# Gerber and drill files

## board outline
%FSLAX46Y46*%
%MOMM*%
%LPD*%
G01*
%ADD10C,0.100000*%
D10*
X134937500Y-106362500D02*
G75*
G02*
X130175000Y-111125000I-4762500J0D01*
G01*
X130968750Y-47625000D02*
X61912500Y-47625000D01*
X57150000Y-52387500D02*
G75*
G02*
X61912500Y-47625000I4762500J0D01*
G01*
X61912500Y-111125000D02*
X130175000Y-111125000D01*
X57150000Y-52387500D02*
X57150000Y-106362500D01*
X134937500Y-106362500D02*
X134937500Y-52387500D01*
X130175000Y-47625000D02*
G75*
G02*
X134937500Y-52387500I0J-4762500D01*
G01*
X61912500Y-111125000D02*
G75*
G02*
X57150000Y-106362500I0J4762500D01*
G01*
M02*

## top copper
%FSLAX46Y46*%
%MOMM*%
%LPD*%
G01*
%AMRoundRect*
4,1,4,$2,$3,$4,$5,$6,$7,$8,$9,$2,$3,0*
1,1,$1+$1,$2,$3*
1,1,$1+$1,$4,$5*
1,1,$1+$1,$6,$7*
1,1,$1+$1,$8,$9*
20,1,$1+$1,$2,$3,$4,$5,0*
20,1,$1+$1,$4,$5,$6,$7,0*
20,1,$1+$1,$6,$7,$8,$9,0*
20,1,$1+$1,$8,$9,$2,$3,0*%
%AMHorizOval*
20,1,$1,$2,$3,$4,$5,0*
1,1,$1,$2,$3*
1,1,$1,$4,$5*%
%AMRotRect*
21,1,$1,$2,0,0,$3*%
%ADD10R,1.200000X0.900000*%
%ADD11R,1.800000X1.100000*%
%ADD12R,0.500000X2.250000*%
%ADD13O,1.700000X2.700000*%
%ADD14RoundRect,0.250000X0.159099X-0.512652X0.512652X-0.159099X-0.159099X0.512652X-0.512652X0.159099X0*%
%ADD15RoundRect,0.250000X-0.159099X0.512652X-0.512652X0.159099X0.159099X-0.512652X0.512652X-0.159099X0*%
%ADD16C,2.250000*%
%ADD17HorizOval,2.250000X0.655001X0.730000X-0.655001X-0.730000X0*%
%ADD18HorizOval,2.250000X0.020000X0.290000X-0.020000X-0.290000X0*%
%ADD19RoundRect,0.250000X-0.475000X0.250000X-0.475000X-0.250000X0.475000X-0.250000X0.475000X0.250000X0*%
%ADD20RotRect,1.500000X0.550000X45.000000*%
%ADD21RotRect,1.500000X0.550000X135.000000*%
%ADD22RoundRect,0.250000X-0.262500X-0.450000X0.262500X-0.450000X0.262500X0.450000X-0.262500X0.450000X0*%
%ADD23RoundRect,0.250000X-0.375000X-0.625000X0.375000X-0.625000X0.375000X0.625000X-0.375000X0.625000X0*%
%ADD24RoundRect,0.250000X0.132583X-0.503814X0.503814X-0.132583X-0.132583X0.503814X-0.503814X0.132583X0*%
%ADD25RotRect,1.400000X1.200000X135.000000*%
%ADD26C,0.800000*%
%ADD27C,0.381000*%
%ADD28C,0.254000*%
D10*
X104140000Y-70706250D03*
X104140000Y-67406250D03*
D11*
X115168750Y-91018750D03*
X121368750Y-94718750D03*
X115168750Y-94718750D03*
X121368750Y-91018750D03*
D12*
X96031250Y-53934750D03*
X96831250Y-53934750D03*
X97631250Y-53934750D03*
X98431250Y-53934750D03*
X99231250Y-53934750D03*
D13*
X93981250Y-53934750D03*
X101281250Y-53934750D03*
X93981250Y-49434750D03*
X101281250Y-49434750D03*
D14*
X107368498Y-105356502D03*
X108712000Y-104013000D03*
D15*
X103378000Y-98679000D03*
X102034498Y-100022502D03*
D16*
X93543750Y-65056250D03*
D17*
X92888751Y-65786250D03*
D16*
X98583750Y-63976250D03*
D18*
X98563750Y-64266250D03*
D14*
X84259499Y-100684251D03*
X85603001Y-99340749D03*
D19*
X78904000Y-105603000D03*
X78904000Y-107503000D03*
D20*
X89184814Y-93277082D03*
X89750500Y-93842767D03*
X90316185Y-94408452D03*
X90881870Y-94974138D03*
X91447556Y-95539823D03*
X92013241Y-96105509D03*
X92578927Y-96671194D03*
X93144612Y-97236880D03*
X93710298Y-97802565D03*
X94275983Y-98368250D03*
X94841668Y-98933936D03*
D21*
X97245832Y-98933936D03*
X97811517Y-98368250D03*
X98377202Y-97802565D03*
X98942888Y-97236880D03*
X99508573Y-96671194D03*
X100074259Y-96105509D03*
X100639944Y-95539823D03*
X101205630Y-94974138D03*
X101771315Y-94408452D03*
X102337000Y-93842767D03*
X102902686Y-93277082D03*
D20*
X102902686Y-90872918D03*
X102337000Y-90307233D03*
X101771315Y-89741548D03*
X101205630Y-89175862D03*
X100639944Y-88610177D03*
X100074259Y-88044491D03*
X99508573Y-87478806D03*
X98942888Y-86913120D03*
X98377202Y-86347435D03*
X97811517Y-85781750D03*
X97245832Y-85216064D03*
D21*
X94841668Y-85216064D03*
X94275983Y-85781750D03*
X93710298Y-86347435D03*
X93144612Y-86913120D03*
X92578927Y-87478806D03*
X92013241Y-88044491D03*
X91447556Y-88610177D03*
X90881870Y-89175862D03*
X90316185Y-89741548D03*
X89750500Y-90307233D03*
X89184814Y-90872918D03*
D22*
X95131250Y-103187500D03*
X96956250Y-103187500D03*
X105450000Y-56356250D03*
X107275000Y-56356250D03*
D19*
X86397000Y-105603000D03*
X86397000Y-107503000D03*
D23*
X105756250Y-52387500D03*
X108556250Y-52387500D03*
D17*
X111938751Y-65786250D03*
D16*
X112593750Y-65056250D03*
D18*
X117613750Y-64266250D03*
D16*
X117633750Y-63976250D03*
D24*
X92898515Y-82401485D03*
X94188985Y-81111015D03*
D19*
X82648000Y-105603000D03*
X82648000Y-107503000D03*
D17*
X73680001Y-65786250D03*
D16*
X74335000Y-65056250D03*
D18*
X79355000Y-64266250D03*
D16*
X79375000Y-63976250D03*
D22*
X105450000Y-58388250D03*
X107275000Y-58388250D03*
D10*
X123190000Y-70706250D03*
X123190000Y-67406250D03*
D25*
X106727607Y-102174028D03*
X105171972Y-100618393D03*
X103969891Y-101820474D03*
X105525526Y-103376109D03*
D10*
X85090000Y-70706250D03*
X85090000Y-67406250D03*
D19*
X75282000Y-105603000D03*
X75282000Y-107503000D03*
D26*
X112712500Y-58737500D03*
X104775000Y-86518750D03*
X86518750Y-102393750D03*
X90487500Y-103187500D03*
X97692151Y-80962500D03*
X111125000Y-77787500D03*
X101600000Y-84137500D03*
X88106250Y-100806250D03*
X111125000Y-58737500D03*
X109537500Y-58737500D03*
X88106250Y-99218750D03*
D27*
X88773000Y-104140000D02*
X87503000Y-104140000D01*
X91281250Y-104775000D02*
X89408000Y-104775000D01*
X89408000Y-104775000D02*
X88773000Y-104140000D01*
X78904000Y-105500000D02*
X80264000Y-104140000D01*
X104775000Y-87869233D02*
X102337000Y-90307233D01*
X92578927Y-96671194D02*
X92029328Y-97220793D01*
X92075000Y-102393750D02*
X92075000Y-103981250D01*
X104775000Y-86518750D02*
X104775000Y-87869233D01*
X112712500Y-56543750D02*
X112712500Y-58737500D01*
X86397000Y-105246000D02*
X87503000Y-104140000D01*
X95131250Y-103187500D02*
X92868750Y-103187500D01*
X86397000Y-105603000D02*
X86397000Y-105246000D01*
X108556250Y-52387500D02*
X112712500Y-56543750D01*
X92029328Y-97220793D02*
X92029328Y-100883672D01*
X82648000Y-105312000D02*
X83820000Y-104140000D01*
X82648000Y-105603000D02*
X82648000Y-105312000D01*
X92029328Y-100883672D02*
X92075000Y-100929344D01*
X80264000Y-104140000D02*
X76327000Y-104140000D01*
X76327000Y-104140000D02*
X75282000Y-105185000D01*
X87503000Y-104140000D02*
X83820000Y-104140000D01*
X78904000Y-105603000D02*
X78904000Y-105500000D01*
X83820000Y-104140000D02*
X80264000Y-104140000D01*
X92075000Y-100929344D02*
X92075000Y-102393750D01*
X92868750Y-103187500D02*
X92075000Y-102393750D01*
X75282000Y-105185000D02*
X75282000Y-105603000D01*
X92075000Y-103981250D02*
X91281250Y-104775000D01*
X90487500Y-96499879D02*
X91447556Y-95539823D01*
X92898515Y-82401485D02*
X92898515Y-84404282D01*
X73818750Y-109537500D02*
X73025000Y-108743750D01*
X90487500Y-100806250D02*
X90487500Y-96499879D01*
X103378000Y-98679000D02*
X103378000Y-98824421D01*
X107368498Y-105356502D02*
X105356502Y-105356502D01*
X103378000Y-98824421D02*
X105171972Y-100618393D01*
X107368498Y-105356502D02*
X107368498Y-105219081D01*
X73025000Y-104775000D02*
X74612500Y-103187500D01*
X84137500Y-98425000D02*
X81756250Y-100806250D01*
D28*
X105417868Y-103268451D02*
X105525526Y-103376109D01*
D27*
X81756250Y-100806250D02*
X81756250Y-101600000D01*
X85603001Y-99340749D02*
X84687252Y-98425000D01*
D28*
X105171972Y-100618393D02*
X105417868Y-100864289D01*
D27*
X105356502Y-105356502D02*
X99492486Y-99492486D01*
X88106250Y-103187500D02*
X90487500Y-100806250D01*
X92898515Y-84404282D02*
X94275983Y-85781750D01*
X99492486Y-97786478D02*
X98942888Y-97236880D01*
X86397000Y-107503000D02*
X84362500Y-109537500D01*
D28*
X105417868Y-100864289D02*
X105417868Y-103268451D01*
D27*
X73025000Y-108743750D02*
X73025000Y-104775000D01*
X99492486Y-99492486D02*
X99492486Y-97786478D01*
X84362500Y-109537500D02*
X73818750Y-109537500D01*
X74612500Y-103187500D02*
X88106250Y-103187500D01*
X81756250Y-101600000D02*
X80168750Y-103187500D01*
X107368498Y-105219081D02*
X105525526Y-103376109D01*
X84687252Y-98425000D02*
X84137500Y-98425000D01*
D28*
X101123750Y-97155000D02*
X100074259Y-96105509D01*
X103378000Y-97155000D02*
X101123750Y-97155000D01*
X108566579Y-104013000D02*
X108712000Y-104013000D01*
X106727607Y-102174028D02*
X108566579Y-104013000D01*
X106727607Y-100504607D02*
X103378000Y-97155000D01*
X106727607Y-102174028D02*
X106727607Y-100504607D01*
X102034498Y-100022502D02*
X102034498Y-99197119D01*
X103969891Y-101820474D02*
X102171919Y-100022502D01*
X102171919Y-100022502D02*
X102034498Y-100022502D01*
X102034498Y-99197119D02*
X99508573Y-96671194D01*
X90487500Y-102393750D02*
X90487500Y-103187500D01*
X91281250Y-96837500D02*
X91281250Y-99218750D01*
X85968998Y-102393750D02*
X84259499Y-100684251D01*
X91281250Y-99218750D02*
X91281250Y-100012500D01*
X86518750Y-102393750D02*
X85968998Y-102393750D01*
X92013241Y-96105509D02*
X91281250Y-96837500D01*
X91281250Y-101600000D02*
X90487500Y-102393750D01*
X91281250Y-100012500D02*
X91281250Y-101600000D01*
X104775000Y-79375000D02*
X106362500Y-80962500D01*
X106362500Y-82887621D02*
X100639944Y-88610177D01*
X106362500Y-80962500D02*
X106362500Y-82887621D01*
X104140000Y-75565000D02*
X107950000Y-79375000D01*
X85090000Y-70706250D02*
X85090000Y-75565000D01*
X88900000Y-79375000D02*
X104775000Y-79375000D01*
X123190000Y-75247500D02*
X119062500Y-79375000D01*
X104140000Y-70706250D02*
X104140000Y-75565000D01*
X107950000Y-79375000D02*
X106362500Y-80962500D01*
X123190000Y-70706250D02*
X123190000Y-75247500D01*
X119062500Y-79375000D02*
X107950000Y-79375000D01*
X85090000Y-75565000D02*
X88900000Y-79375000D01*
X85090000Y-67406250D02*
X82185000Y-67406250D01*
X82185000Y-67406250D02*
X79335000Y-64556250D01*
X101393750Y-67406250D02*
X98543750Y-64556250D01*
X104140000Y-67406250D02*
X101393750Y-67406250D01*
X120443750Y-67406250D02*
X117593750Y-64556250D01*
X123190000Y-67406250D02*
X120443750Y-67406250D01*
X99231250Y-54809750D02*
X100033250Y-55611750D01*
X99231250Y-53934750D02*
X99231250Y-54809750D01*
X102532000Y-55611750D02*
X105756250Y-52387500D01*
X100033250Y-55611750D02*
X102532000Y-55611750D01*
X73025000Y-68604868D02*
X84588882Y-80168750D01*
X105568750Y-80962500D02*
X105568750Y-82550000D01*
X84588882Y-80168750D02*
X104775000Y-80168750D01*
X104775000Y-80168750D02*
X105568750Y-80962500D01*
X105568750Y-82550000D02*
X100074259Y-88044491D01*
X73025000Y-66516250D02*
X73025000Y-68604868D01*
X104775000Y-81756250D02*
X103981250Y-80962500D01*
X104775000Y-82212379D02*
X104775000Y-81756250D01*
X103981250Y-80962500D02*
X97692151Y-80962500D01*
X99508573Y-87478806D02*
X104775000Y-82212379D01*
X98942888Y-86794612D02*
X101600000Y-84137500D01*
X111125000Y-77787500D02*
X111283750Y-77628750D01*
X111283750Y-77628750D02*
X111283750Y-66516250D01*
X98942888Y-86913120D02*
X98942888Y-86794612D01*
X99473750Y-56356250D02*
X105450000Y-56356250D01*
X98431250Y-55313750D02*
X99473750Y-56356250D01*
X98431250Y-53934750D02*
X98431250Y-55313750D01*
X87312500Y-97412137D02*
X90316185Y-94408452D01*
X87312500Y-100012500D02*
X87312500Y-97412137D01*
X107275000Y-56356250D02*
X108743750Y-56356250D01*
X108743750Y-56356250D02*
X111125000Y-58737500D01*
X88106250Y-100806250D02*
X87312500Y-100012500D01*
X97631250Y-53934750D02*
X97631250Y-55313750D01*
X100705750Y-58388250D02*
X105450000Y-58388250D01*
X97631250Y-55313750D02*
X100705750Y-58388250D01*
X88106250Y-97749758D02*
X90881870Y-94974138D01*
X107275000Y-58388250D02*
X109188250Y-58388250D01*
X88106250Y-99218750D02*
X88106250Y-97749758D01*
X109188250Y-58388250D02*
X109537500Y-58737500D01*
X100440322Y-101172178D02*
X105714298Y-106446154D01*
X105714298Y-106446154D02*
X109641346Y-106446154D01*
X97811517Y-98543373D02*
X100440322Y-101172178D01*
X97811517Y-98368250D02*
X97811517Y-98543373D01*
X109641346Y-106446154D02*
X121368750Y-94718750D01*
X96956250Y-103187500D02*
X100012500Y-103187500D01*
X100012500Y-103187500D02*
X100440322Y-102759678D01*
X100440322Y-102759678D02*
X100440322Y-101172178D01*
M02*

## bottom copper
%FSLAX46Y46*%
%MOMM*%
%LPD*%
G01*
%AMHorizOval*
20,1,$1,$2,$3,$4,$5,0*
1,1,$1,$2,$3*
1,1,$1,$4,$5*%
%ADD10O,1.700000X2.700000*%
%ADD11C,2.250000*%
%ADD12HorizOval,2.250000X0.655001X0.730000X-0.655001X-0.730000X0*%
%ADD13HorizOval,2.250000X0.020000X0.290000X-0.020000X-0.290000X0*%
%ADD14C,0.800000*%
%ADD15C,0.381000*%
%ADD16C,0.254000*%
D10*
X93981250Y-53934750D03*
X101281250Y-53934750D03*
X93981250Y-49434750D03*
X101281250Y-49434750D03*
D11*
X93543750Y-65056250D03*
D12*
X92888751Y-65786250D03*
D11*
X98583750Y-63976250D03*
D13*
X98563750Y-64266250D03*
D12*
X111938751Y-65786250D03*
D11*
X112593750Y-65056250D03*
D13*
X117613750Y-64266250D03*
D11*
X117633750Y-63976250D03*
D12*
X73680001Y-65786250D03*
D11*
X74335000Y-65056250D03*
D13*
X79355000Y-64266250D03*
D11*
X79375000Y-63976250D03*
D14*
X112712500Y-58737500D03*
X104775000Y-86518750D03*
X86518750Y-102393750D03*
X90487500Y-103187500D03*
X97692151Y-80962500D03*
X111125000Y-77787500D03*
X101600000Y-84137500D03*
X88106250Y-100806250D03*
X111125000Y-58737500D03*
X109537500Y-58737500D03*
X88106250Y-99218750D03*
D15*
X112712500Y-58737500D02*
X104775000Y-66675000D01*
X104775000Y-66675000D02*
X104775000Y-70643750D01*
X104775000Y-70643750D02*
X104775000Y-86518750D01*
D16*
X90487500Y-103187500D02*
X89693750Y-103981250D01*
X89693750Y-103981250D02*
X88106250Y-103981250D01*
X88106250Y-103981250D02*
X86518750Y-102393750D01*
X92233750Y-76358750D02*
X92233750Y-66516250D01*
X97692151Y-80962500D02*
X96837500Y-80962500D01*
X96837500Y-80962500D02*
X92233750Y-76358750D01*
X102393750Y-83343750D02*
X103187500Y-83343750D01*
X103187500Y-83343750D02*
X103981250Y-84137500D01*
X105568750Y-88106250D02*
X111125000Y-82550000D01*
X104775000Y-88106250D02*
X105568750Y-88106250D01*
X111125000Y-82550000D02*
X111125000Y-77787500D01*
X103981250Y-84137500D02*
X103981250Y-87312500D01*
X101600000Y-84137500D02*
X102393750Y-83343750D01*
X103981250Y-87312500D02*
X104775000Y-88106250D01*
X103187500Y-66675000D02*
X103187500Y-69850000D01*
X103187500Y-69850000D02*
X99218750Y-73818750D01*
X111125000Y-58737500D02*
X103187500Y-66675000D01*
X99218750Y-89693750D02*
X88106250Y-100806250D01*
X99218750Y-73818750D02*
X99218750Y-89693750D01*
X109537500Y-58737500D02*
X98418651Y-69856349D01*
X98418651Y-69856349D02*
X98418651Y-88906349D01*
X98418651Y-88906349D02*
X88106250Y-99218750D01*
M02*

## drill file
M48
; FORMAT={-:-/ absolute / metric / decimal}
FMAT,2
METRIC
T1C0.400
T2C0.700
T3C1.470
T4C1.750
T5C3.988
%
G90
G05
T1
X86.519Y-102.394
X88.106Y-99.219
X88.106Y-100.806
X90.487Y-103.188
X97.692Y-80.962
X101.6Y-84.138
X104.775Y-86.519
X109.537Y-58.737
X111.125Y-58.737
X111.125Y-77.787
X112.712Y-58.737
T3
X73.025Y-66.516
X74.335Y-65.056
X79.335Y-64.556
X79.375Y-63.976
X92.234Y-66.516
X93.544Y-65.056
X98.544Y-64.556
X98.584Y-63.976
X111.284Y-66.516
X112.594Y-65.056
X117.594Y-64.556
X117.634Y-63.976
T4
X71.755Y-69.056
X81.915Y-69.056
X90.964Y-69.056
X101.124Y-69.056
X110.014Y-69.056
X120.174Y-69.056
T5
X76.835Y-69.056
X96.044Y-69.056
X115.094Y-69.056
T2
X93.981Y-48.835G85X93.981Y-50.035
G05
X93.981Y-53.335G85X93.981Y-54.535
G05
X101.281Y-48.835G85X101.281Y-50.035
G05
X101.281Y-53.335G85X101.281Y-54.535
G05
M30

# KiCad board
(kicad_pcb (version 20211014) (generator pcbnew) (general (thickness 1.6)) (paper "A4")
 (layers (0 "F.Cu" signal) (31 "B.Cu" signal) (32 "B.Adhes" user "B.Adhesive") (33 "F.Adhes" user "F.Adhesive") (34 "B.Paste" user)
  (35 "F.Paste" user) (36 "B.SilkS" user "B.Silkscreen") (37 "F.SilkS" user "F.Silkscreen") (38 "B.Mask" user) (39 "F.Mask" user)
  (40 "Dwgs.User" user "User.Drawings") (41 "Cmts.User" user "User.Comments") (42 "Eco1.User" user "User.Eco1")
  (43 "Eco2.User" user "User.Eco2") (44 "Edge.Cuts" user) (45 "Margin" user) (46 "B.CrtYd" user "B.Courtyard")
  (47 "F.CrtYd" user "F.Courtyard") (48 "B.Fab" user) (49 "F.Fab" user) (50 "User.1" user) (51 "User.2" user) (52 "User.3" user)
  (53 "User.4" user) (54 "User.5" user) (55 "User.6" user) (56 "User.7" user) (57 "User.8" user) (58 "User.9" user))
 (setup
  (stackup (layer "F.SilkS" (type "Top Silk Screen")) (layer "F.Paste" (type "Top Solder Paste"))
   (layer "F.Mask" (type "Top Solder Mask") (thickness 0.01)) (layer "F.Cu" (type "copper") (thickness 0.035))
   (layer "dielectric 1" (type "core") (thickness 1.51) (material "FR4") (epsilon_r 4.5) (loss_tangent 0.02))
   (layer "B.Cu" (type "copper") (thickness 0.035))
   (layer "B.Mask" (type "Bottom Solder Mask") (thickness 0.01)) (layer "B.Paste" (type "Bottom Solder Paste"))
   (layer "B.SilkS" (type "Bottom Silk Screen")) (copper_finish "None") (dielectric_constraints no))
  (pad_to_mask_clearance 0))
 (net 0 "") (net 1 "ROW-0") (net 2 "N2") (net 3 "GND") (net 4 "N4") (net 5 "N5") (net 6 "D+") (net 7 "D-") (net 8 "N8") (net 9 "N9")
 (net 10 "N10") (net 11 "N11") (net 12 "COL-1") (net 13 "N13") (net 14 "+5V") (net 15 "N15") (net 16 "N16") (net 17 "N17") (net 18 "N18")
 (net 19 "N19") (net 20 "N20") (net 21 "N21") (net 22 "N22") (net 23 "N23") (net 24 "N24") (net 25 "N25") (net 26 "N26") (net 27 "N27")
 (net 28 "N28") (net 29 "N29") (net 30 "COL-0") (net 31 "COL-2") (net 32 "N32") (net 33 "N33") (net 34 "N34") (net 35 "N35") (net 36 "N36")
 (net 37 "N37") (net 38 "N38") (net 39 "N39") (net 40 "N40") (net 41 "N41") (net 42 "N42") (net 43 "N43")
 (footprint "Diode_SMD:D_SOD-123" (layer "F.Cu") (at 104.14 69.05625 90)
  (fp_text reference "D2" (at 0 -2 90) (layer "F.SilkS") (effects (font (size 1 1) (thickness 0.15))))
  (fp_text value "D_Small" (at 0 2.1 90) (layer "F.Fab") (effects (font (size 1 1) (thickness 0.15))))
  (pad "1" smd rect (at -1.65 0 90) (size 0.9 1.2) (layers "F.Cu" "F.Paste" "F.Mask") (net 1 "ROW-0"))
  (pad "2" smd rect (at 1.65 0 90) (size 0.9 1.2) (layers "F.Cu" "F.Paste" "F.Mask") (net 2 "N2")))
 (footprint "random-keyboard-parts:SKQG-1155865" (layer "F.Cu") (at 118.26875 92.86875 180)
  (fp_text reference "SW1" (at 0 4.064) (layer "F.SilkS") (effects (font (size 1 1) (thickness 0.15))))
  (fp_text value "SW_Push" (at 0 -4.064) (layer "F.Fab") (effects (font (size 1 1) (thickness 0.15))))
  (pad "1" smd rect locked (at 3.1 1.85 180) (size 1.8 1.1) (layers "F.Cu" "F.Paste" "F.Mask") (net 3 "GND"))
  (pad "2" smd rect locked (at -3.1 -1.85 180) (size 1.8 1.1) (layers "F.Cu" "F.Paste" "F.Mask") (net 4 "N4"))
  (pad "3" smd rect locked (at 3.1 -1.85 180) (size 1.8 1.1) (layers "F.Cu" "F.Paste" "F.Mask"))
  (pad "4" smd rect locked (at -3.1 1.85 180) (size 1.8 1.1) (layers "F.Cu" "F.Paste" "F.Mask")))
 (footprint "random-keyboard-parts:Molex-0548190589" (layer "F.Cu") (at 97.63125 49.43475 -90)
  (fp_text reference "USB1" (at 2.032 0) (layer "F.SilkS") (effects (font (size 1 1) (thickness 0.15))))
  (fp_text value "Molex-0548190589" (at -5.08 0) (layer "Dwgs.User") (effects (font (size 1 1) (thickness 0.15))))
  (pad "1" smd rect locked (at 4.5 1.6 270) (size 2.25 0.5) (layers "F.Cu" "F.Paste" "F.Mask") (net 3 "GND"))
  (pad "2" smd rect locked (at 4.5 0.8 270) (size 2.25 0.5) (layers "F.Cu" "F.Paste" "F.Mask") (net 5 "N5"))
  (pad "3" smd rect locked (at 4.5 0 270) (size 2.25 0.5) (layers "F.Cu" "F.Paste" "F.Mask") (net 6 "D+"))
  (pad "4" smd rect locked (at 4.5 -0.8 270) (size 2.25 0.5) (layers "F.Cu" "F.Paste" "F.Mask") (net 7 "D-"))
  (pad "5" smd rect locked (at 4.5 -1.6 270) (size 2.25 0.5) (layers "F.Cu" "F.Paste" "F.Mask") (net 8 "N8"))
  (pad "6" thru_hole oval locked (at 4.5 3.65 270) (size 2.7 1.7) (drill oval 1.9 0.7) (layers *.Cu *.Mask) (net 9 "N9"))
  (pad "6" thru_hole oval locked (at 4.5 -3.65 270) (size 2.7 1.7) (drill oval 1.9 0.7) (layers *.Cu *.Mask) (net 9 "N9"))
  (pad "6" thru_hole oval locked (at 0 3.65 270) (size 2.7 1.7) (drill oval 1.9 0.7) (layers *.Cu *.Mask) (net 9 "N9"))
  (pad "6" thru_hole oval locked (at 0 -3.65 270) (size 2.7 1.7) (drill oval 1.9 0.7) (layers *.Cu *.Mask) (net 9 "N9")))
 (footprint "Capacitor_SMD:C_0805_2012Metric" (layer "F.Cu") (at 108.040249 104.684751 45)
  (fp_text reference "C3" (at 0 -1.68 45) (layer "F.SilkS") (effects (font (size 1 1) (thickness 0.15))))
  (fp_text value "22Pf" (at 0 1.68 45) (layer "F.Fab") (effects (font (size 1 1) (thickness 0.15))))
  (pad "1" smd roundrect (at -0.95 0 45) (size 1 1.45) (layers "F.Cu" "F.Paste" "F.Mask") (roundrect_rratio 0.25) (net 3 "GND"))
  (pad "2" smd roundrect (at 0.95 0 45) (size 1 1.45) (layers "F.Cu" "F.Paste" "F.Mask") (roundrect_rratio 0.25) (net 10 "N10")))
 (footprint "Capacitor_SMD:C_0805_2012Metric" (layer "F.Cu") (at 102.706249 99.350751 -135)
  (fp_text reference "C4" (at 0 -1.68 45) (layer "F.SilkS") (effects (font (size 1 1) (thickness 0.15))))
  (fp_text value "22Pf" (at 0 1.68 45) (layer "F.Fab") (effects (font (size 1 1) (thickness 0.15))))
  (pad "1" smd roundrect (at -0.95 0 225) (size 1 1.45) (layers "F.Cu" "F.Paste" "F.Mask") (roundrect_rratio 0.25) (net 3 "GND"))
  (pad "2" smd roundrect (at 0.95 0 225) (size 1 1.45) (layers "F.Cu" "F.Paste" "F.Mask") (roundrect_rratio 0.25) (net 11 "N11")))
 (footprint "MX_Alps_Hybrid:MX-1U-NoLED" (layer "F.Cu") (at 96.04375 69.05625)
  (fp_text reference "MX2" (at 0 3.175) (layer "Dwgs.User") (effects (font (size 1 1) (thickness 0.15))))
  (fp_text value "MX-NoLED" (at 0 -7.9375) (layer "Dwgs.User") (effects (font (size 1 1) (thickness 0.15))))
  (pad "" np_thru_hole circle locked (at -5.08 0 48.0996) (size 1.75 1.75) (drill 1.75) (layers *.Cu *.Mask))
  (pad "" np_thru_hole circle locked (at 0 0) (size 3.9878 3.9878) (drill 3.9878) (layers *.Cu *.Mask))
  (pad "" np_thru_hole circle locked (at 5.08 0 48.0996) (size 1.75 1.75) (drill 1.75) (layers *.Cu *.Mask))
  (pad "1" thru_hole circle locked (at -2.5 -4) (size 2.25 2.25) (drill 1.47) (layers *.Cu "B.Mask") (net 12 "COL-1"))
  (pad "1" thru_hole oval locked (at -3.81 -2.54 48.0996) (size 4.211556 2.25) (drill 1.47 (offset 0.980778 0)) (layers *.Cu "B.Mask")
   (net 12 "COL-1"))
  (pad "2" thru_hole circle locked (at 2.54 -5.08) (size 2.25 2.25) (drill 1.47) (layers *.Cu "B.Mask") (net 2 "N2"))
  (pad "2" thru_hole oval locked (at 2.5 -4.5 86.0548) (size 2.831378 2.25) (drill 1.47 (offset 0.290689 0)) (layers *.Cu "B.Mask")
   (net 2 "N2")))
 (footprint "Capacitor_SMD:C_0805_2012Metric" (layer "F.Cu") (at 84.93125 100.0125 45)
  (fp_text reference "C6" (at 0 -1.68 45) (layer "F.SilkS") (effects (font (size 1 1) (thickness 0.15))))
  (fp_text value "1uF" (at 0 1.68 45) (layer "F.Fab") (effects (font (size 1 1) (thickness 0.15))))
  (pad "1" smd roundrect (at -0.95 0 45) (size 1 1.45) (layers "F.Cu" "F.Paste" "F.Mask") (roundrect_rratio 0.25) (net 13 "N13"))
  (pad "2" smd roundrect (at 0.95 0 45) (size 1 1.45) (layers "F.Cu" "F.Paste" "F.Mask") (roundrect_rratio 0.25) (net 3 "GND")))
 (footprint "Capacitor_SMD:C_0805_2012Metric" (layer "F.Cu") (at 78.904 106.553 -90)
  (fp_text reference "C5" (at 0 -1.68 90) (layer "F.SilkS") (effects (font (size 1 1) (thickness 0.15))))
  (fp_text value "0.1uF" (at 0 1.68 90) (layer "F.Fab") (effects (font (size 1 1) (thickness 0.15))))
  (pad "1" smd roundrect (at -0.95 0 270) (size 1 1.45) (layers "F.Cu" "F.Paste" "F.Mask") (roundrect_rratio 0.25) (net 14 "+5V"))
  (pad "2" smd roundrect (at 0.95 0 270) (size 1 1.45) (layers "F.Cu" "F.Paste" "F.Mask") (roundrect_rratio 0.25) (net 3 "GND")))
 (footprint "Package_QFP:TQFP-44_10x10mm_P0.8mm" (layer "F.Cu") (at 96.04375 92.075 45)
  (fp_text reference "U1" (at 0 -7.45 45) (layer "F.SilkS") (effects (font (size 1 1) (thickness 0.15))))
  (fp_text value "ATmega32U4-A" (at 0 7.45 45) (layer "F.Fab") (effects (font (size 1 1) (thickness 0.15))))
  (pad "1" smd rect (at -5.7 -4 45) (size 1.5 0.55) (layers "F.Cu" "F.Paste" "F.Mask") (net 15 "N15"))
  (pad "2" smd rect (at -5.7 -3.2 45) (size 1.5 0.55) (layers "F.Cu" "F.Paste" "F.Mask") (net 14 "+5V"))
  (pad "3" smd rect (at -5.7 -2.4 45) (size 1.5 0.55) (layers "F.Cu" "F.Paste" "F.Mask") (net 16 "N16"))
  (pad "4" smd rect (at -5.7 -1.6 45) (size 1.5 0.55) (layers "F.Cu" "F.Paste" "F.Mask") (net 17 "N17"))
  (pad "5" smd rect (at -5.7 -0.8 45) (size 1.5 0.55) (layers "F.Cu" "F.Paste" "F.Mask") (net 3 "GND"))
  (pad "6" smd rect (at -5.7 0 45) (size 1.5 0.55) (layers "F.Cu" "F.Paste" "F.Mask") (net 13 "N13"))
  (pad "7" smd rect (at -5.7 0.8 45) (size 1.5 0.55) (layers "F.Cu" "F.Paste" "F.Mask") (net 14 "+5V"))
  (pad "8" smd rect (at -5.7 1.6 45) (size 1.5 0.55) (layers "F.Cu" "F.Paste" "F.Mask") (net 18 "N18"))
  (pad "9" smd rect (at -5.7 2.4 45) (size 1.5 0.55) (layers "F.Cu" "F.Paste" "F.Mask") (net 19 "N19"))
  (pad "10" smd rect (at -5.7 3.2 45) (size 1.5 0.55) (layers "F.Cu" "F.Paste" "F.Mask") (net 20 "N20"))
  (pad "11" smd rect (at -5.7 4 45) (size 1.5 0.55) (layers "F.Cu" "F.Paste" "F.Mask") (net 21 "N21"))
  (pad "12" smd rect (at -4 5.7 135) (size 1.5 0.55) (layers "F.Cu" "F.Paste" "F.Mask") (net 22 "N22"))
  (pad "13" smd rect (at -3.2 5.7 135) (size 1.5 0.55) (layers "F.Cu" "F.Paste" "F.Mask") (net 4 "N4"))
  (pad "14" smd rect (at -2.4 5.7 135) (size 1.5 0.55) (layers "F.Cu" "F.Paste" "F.Mask") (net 14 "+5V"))
  (pad "15" smd rect (at -1.6 5.7 135) (size 1.5 0.55) (layers "F.Cu" "F.Paste" "F.Mask") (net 3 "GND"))
  (pad "16" smd rect (at -0.8 5.7 135) (size 1.5 0.55) (layers "F.Cu" "F.Paste" "F.Mask") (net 11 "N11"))
  (pad "17" smd rect (at 0 5.7 135) (size 1.5 0.55) (layers "F.Cu" "F.Paste" "F.Mask") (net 10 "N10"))
  (pad "18" smd rect (at 0.8 5.7 135) (size 1.5 0.55) (layers "F.Cu" "F.Paste" "F.Mask") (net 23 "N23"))
  (pad "19" smd rect (at 1.6 5.7 135) (size 1.5 0.55) (layers "F.Cu" "F.Paste" "F.Mask") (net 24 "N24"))
  (pad "20" smd rect (at 2.4 5.7 135) (size 1.5 0.55) (layers "F.Cu" "F.Paste" "F.Mask") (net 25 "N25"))
  (pad "21" smd rect (at 3.2 5.7 135) (size 1.5 0.55) (layers "F.Cu" "F.Paste" "F.Mask") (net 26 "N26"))
  (pad "22" smd rect (at 4 5.7 135) (size 1.5 0.55) (layers "F.Cu" "F.Paste" "F.Mask") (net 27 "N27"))
  (pad "23" smd rect (at 5.7 4 45) (size 1.5 0.55) (layers "F.Cu" "F.Paste" "F.Mask") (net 3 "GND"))
  (pad "24" smd rect (at 5.7 3.2 45) (size 1.5 0.55) (layers "F.Cu" "F.Paste" "F.Mask") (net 14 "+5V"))
  (pad "25" smd rect (at 5.7 2.4 45) (size 1.5 0.55) (layers "F.Cu" "F.Paste" "F.Mask") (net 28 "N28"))
  (pad "26" smd rect (at 5.7 1.6 45) (size 1.5 0.55) (layers "F.Cu" "F.Paste" "F.Mask") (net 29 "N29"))
  (pad "27" smd rect (at 5.7 0.8 45) (size 1.5 0.55) (layers "F.Cu" "F.Paste" "F.Mask") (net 1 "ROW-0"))
  (pad "28" smd rect (at 5.7 0 45) (size 1.5 0.55) (layers "F.Cu" "F.Paste" "F.Mask") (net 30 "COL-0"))
  (pad "29" smd rect (at 5.7 -0.8 45) (size 1.5 0.55) (layers "F.Cu" "F.Paste" "F.Mask") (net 12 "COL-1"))
  (pad "30" smd rect (at 5.7 -1.6 45) (size 1.5 0.55) (layers "F.Cu" "F.Paste" "F.Mask") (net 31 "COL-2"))
  (pad "31" smd rect (at 5.7 -2.4 45) (size 1.5 0.55) (layers "F.Cu" "F.Paste" "F.Mask") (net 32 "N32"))
  (pad "32" smd rect (at 5.7 -3.2 45) (size 1.5 0.55) (layers "F.Cu" "F.Paste" "F.Mask") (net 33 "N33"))
  (pad "33" smd rect (at 5.7 -4 45) (size 1.5 0.55) (layers "F.Cu" "F.Paste" "F.Mask") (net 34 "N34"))
  (pad "34" smd rect (at 4 -5.7 135) (size 1.5 0.55) (layers "F.Cu" "F.Paste" "F.Mask") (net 14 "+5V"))
  (pad "35" smd rect (at 3.2 -5.7 135) (size 1.5 0.55) (layers "F.Cu" "F.Paste" "F.Mask") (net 3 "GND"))
  (pad "36" smd rect (at 2.4 -5.7 135) (size 1.5 0.55) (layers "F.Cu" "F.Paste" "F.Mask") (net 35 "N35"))
  (pad "37" smd rect (at 1.6 -5.7 135) (size 1.5 0.55) (layers "F.Cu" "F.Paste" "F.Mask") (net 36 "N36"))
  (pad "38" smd rect (at 0.8 -5.7 135) (size 1.5 0.55) (layers "F.Cu" "F.Paste" "F.Mask") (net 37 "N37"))
  (pad "39" smd rect (at 0 -5.7 135) (size 1.5 0.55) (layers "F.Cu" "F.Paste" "F.Mask") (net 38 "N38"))
  (pad "40" smd rect (at -0.8 -5.7 135) (size 1.5 0.55) (layers "F.Cu" "F.Paste" "F.Mask") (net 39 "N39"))
  (pad "41" smd rect (at -1.6 -5.7 135) (size 1.5 0.55) (layers "F.Cu" "F.Paste" "F.Mask") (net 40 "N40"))
  (pad "42" smd rect (at -2.4 -5.7 135) (size 1.5 0.55) (layers "F.Cu" "F.Paste" "F.Mask") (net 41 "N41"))
  (pad "43" smd rect (at -3.2 -5.7 135) (size 1.5 0.55) (layers "F.Cu" "F.Paste" "F.Mask") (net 3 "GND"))
  (pad "44" smd rect (at -4 -5.7 135) (size 1.5 0.55) (layers "F.Cu" "F.Paste" "F.Mask") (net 14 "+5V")))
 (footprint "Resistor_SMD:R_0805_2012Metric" (layer "F.Cu") (at 96.04375 103.1875)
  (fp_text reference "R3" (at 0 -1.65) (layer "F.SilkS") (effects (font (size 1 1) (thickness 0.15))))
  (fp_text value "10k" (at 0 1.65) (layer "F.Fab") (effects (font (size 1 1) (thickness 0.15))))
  (pad "1" smd roundrect (at -0.9125 0) (size 1.025 1.4) (layers "F.Cu" "F.Paste" "F.Mask") (roundrect_rratio 0.243902) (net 14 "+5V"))
  (pad "2" smd roundrect (at 0.9125 0) (size 1.025 1.4) (layers "F.Cu" "F.Paste" "F.Mask") (roundrect_rratio 0.243902) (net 4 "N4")))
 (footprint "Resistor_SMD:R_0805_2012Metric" (layer "F.Cu") (at 106.3625 56.35625)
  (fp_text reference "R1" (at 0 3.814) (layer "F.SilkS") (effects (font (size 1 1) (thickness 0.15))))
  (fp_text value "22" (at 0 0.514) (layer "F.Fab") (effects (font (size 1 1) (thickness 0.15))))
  (pad "1" smd roundrect (at -0.9125 0) (size 1.025 1.4) (layers "F.Cu" "F.Paste" "F.Mask") (roundrect_rratio 0.243902) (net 7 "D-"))
  (pad "2" smd roundrect (at 0.9125 0) (size 1.025 1.4) (layers "F.Cu" "F.Paste" "F.Mask") (roundrect_rratio 0.243902) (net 16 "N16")))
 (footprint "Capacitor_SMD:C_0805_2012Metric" (layer "F.Cu") (at 86.397 106.553 -90)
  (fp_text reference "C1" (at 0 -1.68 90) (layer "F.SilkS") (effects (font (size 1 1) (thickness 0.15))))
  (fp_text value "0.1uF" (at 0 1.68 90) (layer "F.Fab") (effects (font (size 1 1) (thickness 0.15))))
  (pad "1" smd roundrect (at -0.95 0 270) (size 1 1.45) (layers "F.Cu" "F.Paste" "F.Mask") (roundrect_rratio 0.25) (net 14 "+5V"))
  (pad "2" smd roundrect (at 0.95 0 270) (size 1 1.45) (layers "F.Cu" "F.Paste" "F.Mask") (roundrect_rratio 0.25) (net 3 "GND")))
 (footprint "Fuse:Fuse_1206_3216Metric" (layer "F.Cu") (at 107.15625 52.3875)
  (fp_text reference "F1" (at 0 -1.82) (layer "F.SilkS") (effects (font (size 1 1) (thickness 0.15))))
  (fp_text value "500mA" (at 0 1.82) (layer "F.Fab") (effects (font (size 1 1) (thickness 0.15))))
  (pad "1" smd roundrect (at -1.4 0) (size 1.25 1.75) (layers "F.Cu" "F.Paste" "F.Mask") (roundrect_rratio 0.2) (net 8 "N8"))
  (pad "2" smd roundrect (at 1.4 0) (size 1.25 1.75) (layers "F.Cu" "F.Paste" "F.Mask") (roundrect_rratio 0.2) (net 14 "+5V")))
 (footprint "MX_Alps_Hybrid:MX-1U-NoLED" (layer "F.Cu") (at 115.09375 69.05625)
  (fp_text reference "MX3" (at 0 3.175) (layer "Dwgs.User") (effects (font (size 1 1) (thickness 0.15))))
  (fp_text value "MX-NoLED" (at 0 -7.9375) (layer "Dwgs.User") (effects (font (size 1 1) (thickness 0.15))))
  (pad "" np_thru_hole circle locked (at -5.08 0 48.0996) (size 1.75 1.75) (drill 1.75) (layers *.Cu *.Mask))
  (pad "" np_thru_hole circle locked (at 5.08 0 48.0996) (size 1.75 1.75) (drill 1.75) (layers *.Cu *.Mask))
  (pad "" np_thru_hole circle locked (at 0 0) (size 3.9878 3.9878) (drill 3.9878) (layers *.Cu *.Mask))
  (pad "1" thru_hole oval locked (at -3.81 -2.54 48.0996) (size 4.211556 2.25) (drill 1.47 (offset 0.980778 0)) (layers *.Cu "B.Mask")
   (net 31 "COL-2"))
  (pad "1" thru_hole circle locked (at -2.5 -4) (size 2.25 2.25) (drill 1.47) (layers *.Cu "B.Mask") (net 31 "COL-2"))
  (pad "2" thru_hole oval locked (at 2.5 -4.5 86.0548) (size 2.831378 2.25) (drill 1.47 (offset 0.290689 0)) (layers *.Cu "B.Mask")
   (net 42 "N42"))
  (pad "2" thru_hole circle locked (at 2.54 -5.08) (size 2.25 2.25) (drill 1.47) (layers *.Cu "B.Mask") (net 42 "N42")))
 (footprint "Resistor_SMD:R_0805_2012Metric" (layer "F.Cu") (at 93.54375 81.75625 45)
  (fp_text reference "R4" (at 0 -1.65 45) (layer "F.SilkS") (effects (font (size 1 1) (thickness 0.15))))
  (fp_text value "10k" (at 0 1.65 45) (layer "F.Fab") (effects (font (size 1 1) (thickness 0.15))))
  (pad "1" smd roundrect (at -0.9125 0 45) (size 1.025 1.4) (layers "F.Cu" "F.Paste" "F.Mask") (roundrect_rratio 0.243902) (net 3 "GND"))
  (pad "2" smd roundrect (at 0.9125 0 45) (size 1.025 1.4) (layers "F.Cu" "F.Paste" "F.Mask") (roundrect_rratio 0.243902) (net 34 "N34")))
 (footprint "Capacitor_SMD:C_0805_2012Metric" (layer "F.Cu") (at 82.648 106.553 -90)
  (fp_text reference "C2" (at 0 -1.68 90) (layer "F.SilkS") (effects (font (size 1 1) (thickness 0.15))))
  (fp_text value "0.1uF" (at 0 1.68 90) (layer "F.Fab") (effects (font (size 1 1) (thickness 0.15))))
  (pad "1" smd roundrect (at -0.95 0 270) (size 1 1.45) (layers "F.Cu" "F.Paste" "F.Mask") (roundrect_rratio 0.25) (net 14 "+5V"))
  (pad "2" smd roundrect (at 0.95 0 270) (size 1 1.45) (layers "F.Cu" "F.Paste" "F.Mask") (roundrect_rratio 0.25) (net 3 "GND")))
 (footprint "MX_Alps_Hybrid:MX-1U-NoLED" (layer "F.Cu") (at 76.835 69.05625)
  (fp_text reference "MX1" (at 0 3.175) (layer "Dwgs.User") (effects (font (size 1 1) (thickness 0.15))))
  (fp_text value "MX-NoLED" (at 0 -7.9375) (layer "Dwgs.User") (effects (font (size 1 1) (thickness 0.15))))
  (pad "" np_thru_hole circle locked (at -5.08 0 48.0996) (size 1.75 1.75) (drill 1.75) (layers *.Cu *.Mask))
  (pad "" np_thru_hole circle locked (at 5.08 0 48.0996) (size 1.75 1.75) (drill 1.75) (layers *.Cu *.Mask))
  (pad "" np_thru_hole circle locked (at 0 0) (size 3.9878 3.9878) (drill 3.9878) (layers *.Cu *.Mask))
  (pad "1" thru_hole oval locked (at -3.81 -2.54 48.0996) (size 4.211556 2.25) (drill 1.47 (offset 0.980778 0)) (layers *.Cu "B.Mask")
   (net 30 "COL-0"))
  (pad "1" thru_hole circle locked (at -2.5 -4) (size 2.25 2.25) (drill 1.47) (layers *.Cu "B.Mask") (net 30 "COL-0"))
  (pad "2" thru_hole oval locked (at 2.5 -4.5 86.0548) (size 2.831378 2.25) (drill 1.47 (offset 0.290689 0)) (layers *.Cu "B.Mask")
   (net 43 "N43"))
  (pad "2" thru_hole circle locked (at 2.54 -5.08) (size 2.25 2.25) (drill 1.47) (layers *.Cu "B.Mask") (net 43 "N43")))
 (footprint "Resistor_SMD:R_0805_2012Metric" (layer "F.Cu") (at 106.3625 58.38825)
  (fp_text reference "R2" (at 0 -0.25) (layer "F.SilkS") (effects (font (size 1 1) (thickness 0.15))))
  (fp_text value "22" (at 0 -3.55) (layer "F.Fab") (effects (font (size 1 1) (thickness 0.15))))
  (pad "1" smd roundrect (at -0.9125 0) (size 1.025 1.4) (layers "F.Cu" "F.Paste" "F.Mask") (roundrect_rratio 0.243902) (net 6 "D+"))
  (pad "2" smd roundrect (at 0.9125 0) (size 1.025 1.4) (layers "F.Cu" "F.Paste" "F.Mask") (roundrect_rratio 0.243902) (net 17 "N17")))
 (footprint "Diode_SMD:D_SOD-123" (layer "F.Cu") (at 123.19 69.05625 90)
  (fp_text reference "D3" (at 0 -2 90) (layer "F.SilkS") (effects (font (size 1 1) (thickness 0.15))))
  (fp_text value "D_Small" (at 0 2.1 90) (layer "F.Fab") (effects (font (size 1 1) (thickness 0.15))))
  (pad "1" smd rect (at -1.65 0 90) (size 0.9 1.2) (layers "F.Cu" "F.Paste" "F.Mask") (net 1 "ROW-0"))
  (pad "2" smd rect (at 1.65 0 90) (size 0.9 1.2) (layers "F.Cu" "F.Paste" "F.Mask") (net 42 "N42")))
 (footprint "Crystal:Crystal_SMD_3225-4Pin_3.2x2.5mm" (layer "F.Cu") (at 105.348749 101.997251 135)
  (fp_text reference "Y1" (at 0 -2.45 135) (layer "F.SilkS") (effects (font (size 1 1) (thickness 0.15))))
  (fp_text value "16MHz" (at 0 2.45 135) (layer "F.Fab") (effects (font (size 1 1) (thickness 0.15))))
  (pad "1" smd rect (at -1.1 0.85 135) (size 1.4 1.2) (layers "F.Cu" "F.Paste" "F.Mask") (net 10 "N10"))
  (pad "2" smd rect (at 1.1 0.85 135) (size 1.4 1.2) (layers "F.Cu" "F.Paste" "F.Mask") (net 3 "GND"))
  (pad "3" smd rect (at 1.1 -0.85 135) (size 1.4 1.2) (layers "F.Cu" "F.Paste" "F.Mask") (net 11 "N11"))
  (pad "4" smd rect (at -1.1 -0.85 135) (size 1.4 1.2) (layers "F.Cu" "F.Paste" "F.Mask") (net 3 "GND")))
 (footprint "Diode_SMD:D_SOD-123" (layer "F.Cu") (at 85.09 69.05625 90)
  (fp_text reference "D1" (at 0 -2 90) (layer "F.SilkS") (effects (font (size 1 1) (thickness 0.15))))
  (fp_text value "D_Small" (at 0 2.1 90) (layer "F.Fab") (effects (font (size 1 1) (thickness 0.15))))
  (pad "1" smd rect (at -1.65 0 90) (size 0.9 1.2) (layers "F.Cu" "F.Paste" "F.Mask") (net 1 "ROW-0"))
  (pad "2" smd rect (at 1.65 0 90) (size 0.9 1.2) (layers "F.Cu" "F.Paste" "F.Mask") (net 43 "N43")))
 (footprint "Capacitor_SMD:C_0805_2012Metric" (layer "F.Cu") (at 75.282 106.553 -90)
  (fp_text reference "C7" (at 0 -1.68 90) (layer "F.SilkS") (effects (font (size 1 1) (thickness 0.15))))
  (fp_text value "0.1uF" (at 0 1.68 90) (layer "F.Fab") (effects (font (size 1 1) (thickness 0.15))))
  (pad "1" smd roundrect (at -0.95 0 270) (size 1 1.45) (layers "F.Cu" "F.Paste" "F.Mask") (roundrect_rratio 0.25) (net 14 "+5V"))
  (pad "2" smd roundrect (at 0.95 0 270) (size 1 1.45) (layers "F.Cu" "F.Paste" "F.Mask") (roundrect_rratio 0.25) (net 3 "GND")))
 (gr_arc (start 134.9375 106.3625) (mid 133.542596 109.730096) (end 130.175 111.125) (layer "Edge.Cuts") (width 0.1))
 (gr_line (start 130.96875 47.625) (end 61.9125 47.625) (layer "Edge.Cuts") (width 0.1))
 (gr_arc (start 57.15 52.3875) (mid 58.544904 49.019904) (end 61.9125 47.625) (layer "Edge.Cuts") (width 0.1))
 (gr_line (start 61.9125 111.125) (end 130.175 111.125) (layer "Edge.Cuts") (width 0.1))
 (gr_line (start 57.15 52.3875) (end 57.15 106.3625) (layer "Edge.Cuts") (width 0.1))
 (gr_line (start 134.9375 106.3625) (end 134.9375 52.3875) (layer "Edge.Cuts") (width 0.1))
 (gr_arc (start 130.175 47.625) (mid 133.542596 49.019904) (end 134.9375 52.3875) (layer "Edge.Cuts") (width 0.1))
 (gr_arc (start 61.9125 111.125) (mid 58.544904 109.730096) (end 57.15 106.3625) (layer "Edge.Cuts") (width 0.1))
 (segment (start 88.773 104.14) (end 87.503 104.14) (width 0.381) (layer "F.Cu") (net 14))
 (segment (start 91.28125 104.775) (end 89.408 104.775) (width 0.381) (layer "F.Cu") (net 14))
 (segment (start 89.408 104.775) (end 88.773 104.14) (width 0.381) (layer "F.Cu") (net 14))
 (segment (start 78.904 105.5) (end 80.264 104.14) (width 0.381) (layer "F.Cu") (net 14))
 (segment (start 104.775 87.869233) (end 102.337 90.307233) (width 0.381) (layer "F.Cu") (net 14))
 (segment (start 92.578927 96.671194) (end 92.029328 97.220793) (width 0.381) (layer "F.Cu") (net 14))
 (segment (start 92.075 102.39375) (end 92.075 103.98125) (width 0.381) (layer "F.Cu") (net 14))
 (segment (start 104.775 86.51875) (end 104.775 87.869233) (width 0.381) (layer "F.Cu") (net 14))
 (segment (start 112.7125 56.54375) (end 112.7125 58.7375) (width 0.381) (layer "F.Cu") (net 14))
 (segment (start 86.397 105.246) (end 87.503 104.14) (width 0.381) (layer "F.Cu") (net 14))
 (segment (start 95.13125 103.1875) (end 92.86875 103.1875) (width 0.381) (layer "F.Cu") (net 14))
 (segment (start 86.397 105.603) (end 86.397 105.246) (width 0.381) (layer "F.Cu") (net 14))
 (segment (start 108.55625 52.3875) (end 112.7125 56.54375) (width 0.381) (layer "F.Cu") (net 14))
 (segment (start 92.029328 97.220793) (end 92.029328 100.883672) (width 0.381) (layer "F.Cu") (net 14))
 (segment (start 82.648 105.312) (end 83.82 104.14) (width 0.381) (layer "F.Cu") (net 14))
 (segment (start 82.648 105.603) (end 82.648 105.312) (width 0.381) (layer "F.Cu") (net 14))
 (segment (start 92.029328 100.883672) (end 92.075 100.929344) (width 0.381) (layer "F.Cu") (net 14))
 (segment (start 80.264 104.14) (end 76.327 104.14) (width 0.381) (layer "F.Cu") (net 14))
 (segment (start 76.327 104.14) (end 75.282 105.185) (width 0.381) (layer "F.Cu") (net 14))
 (segment (start 87.503 104.14) (end 83.82 104.14) (width 0.381) (layer "F.Cu") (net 14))
 (segment (start 78.904 105.603) (end 78.904 105.5) (width 0.381) (layer "F.Cu") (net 14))
 (segment (start 83.82 104.14) (end 80.264 104.14) (width 0.381) (layer "F.Cu") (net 14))
 (segment (start 92.075 100.929344) (end 92.075 102.39375) (width 0.381) (layer "F.Cu") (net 14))
 (segment (start 92.86875 103.1875) (end 92.075 102.39375) (width 0.381) (layer "F.Cu") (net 14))
 (segment (start 75.282 105.185) (end 75.282 105.603) (width 0.381) (layer "F.Cu") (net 14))
 (segment (start 92.075 103.98125) (end 91.28125 104.775) (width 0.381) (layer "F.Cu") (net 14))
 (via (at 112.7125 58.7375) (size 0.8) (drill 0.4) (layers "F.Cu" "B.Cu") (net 14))
 (via (at 104.775 86.51875) (size 0.8) (drill 0.4) (layers "F.Cu" "B.Cu") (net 14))
 (segment (start 112.7125 58.7375) (end 104.775 66.675) (width 0.381) (layer "B.Cu") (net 14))
 (segment (start 104.775 66.675) (end 104.775 70.64375) (width 0.381) (layer "B.Cu") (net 14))
 (segment (start 104.775 70.64375) (end 104.775 86.51875) (width 0.381) (layer "B.Cu") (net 14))
 (segment (start 90.4875 96.499879) (end 91.447556 95.539823) (width 0.381) (layer "F.Cu") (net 3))
 (segment (start 92.898515 82.401485) (end 92.898515 84.404282) (width 0.381) (layer "F.Cu") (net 3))
 (segment (start 73.81875 109.5375) (end 73.025 108.74375) (width 0.381) (layer "F.Cu") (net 3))
 (segment (start 90.4875 100.80625) (end 90.4875 96.499879) (width 0.381) (layer "F.Cu") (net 3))
 (segment (start 103.378 98.679) (end 103.378 98.824421) (width 0.381) (layer "F.Cu") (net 3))
 (segment (start 107.368498 105.356502) (end 105.356502 105.356502) (width 0.381) (layer "F.Cu") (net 3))
 (segment (start 103.378 98.824421) (end 105.171972 100.618393) (width 0.381) (layer "F.Cu") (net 3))
 (segment (start 107.368498 105.356502) (end 107.368498 105.219081) (width 0.381) (layer "F.Cu") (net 3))
 (segment (start 73.025 104.775) (end 74.6125 103.1875) (width 0.381) (layer "F.Cu") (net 3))
 (segment (start 84.1375 98.425) (end 81.75625 100.80625) (width 0.381) (layer "F.Cu") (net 3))
 (segment (start 105.417868 103.268451) (end 105.525526 103.376109) (width 0.254) (layer "F.Cu") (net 3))
 (segment (start 81.75625 100.80625) (end 81.75625 101.6) (width 0.381) (layer "F.Cu") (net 3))
 (segment (start 85.603001 99.340749) (end 84.687252 98.425) (width 0.381) (layer "F.Cu") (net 3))
 (segment (start 105.171972 100.618393) (end 105.417868 100.864289) (width 0.254) (layer "F.Cu") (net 3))
 (segment (start 105.356502 105.356502) (end 99.492486 99.492486) (width 0.381) (layer "F.Cu") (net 3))
 (segment (start 88.10625 103.1875) (end 90.4875 100.80625) (width 0.381) (layer "F.Cu") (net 3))
 (segment (start 92.898515 84.404282) (end 94.275983 85.78175) (width 0.381) (layer "F.Cu") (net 3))
 (segment (start 99.492486 97.786478) (end 98.942888 97.23688) (width 0.381) (layer "F.Cu") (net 3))
 (segment (start 86.397 107.503) (end 84.3625 109.5375) (width 0.381) (layer "F.Cu") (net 3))
 (segment (start 105.417868 100.864289) (end 105.417868 103.268451) (width 0.254) (layer "F.Cu") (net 3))
 (segment (start 73.025 108.74375) (end 73.025 104.775) (width 0.381) (layer "F.Cu") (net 3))
 (segment (start 99.492486 99.492486) (end 99.492486 97.786478) (width 0.381) (layer "F.Cu") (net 3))
 (segment (start 84.3625 109.5375) (end 73.81875 109.5375) (width 0.381) (layer "F.Cu") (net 3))
 (segment (start 74.6125 103.1875) (end 88.10625 103.1875) (width 0.381) (layer "F.Cu") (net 3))
 (segment (start 81.75625 101.6) (end 80.16875 103.1875) (width 0.381) (layer "F.Cu") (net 3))
 (segment (start 107.368498 105.219081) (end 105.525526 103.376109) (width 0.381) (layer "F.Cu") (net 3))
 (segment (start 84.687252 98.425) (end 84.1375 98.425) (width 0.381) (layer "F.Cu") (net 3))
 (segment (start 101.12375 97.155) (end 100.074259 96.105509) (width 0.254) (layer "F.Cu") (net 10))
 (segment (start 103.378 97.155) (end 101.12375 97.155) (width 0.254) (layer "F.Cu") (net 10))
 (segment (start 108.566579 104.013) (end 108.712 104.013) (width 0.254) (layer "F.Cu") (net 10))
 (segment (start 106.727607 102.174028) (end 108.566579 104.013) (width 0.254) (layer "F.Cu") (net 10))
 (segment (start 106.727607 100.504607) (end 103.378 97.155) (width 0.254) (layer "F.Cu") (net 10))
 (segment (start 106.727607 102.174028) (end 106.727607 100.504607) (width 0.254) (layer "F.Cu") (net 10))
 (segment (start 102.034498 100.022502) (end 102.034498 99.197119) (width 0.254) (layer "F.Cu") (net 11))
 (segment (start 103.969891 101.820474) (end 102.171919 100.022502) (width 0.254) (layer "F.Cu") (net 11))
 (segment (start 102.171919 100.022502) (end 102.034498 100.022502) (width 0.254) (layer "F.Cu") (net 11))
 (segment (start 102.034498 99.197119) (end 99.508573 96.671194) (width 0.254) (layer "F.Cu") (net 11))
 (segment (start 90.4875 102.39375) (end 90.4875 103.1875) (width 0.254) (layer "F.Cu") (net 13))
 (segment (start 91.28125 96.8375) (end 91.28125 99.21875) (width 0.254) (layer "F.Cu") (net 13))
 (segment (start 85.968998 102.39375) (end 84.259499 100.684251) (width 0.254) (layer "F.Cu") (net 13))
 (segment (start 91.28125 99.21875) (end 91.28125 100.0125) (width 0.254) (layer "F.Cu") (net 13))
 (segment (start 86.51875 102.39375) (end 85.968998 102.39375) (width 0.254) (layer "F.Cu") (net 13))
 (segment (start 92.013241 96.105509) (end 91.28125 96.8375) (width 0.254) (layer "F.Cu") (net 13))
 (segment (start 91.28125 101.6) (end 90.4875 102.39375) (width 0.254) (layer "F.Cu") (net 13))
 (segment (start 91.28125 100.0125) (end 91.28125 101.6) (width 0.254) (layer "F.Cu") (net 13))
 (via (at 86.51875 102.39375) (size 0.8) (drill 0.4) (layers "F.Cu" "B.Cu") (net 13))
 (via (at 90.4875 103.1875) (size 0.8) (drill 0.4) (layers "F.Cu" "B.Cu") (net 13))
 (segment (start 90.4875 103.1875) (end 89.69375 103.98125) (width 0.254) (layer "B.Cu") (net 13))
 (segment (start 89.69375 103.98125) (end 88.10625 103.98125) (width 0.254) (layer "B.Cu") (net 13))
 (segment (start 88.10625 103.98125) (end 86.51875 102.39375) (width 0.254) (layer "B.Cu") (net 13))
 (segment (start 104.775 79.375) (end 106.3625 80.9625) (width 0.254) (layer "F.Cu") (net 1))
 (segment (start 106.3625 82.887621) (end 100.639944 88.610177) (width 0.254) (layer "F.Cu") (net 1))
 (segment (start 106.3625 80.9625) (end 106.3625 82.887621) (width 0.254) (layer "F.Cu") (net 1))
 (segment (start 104.14 75.565) (end 107.95 79.375) (width 0.254) (layer "F.Cu") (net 1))
 (segment (start 85.09 70.70625) (end 85.09 75.565) (width 0.254) (layer "F.Cu") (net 1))
 (segment (start 88.9 79.375) (end 104.775 79.375) (width 0.254) (layer "F.Cu") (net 1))
 (segment (start 123.19 75.2475) (end 119.0625 79.375) (width 0.254) (layer "F.Cu") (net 1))
 (segment (start 104.14 70.70625) (end 104.14 75.565) (width 0.254) (layer "F.Cu") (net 1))
 (segment (start 107.95 79.375) (end 106.3625 80.9625) (width 0.254) (layer "F.Cu") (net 1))
 (segment (start 123.19 70.70625) (end 123.19 75.2475) (width 0.254) (layer "F.Cu") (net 1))
 (segment (start 119.0625 79.375) (end 107.95 79.375) (width 0.254) (layer "F.Cu") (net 1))
 (segment (start 85.09 75.565) (end 88.9 79.375) (width 0.254) (layer "F.Cu") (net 1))
 (segment (start 85.09 67.40625) (end 82.185 67.40625) (width 0.254) (layer "F.Cu") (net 43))
 (segment (start 82.185 67.40625) (end 79.335 64.55625) (width 0.254) (layer "F.Cu") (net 43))
 (segment (start 101.39375 67.40625) (end 98.54375 64.55625) (width 0.254) (layer "F.Cu") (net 2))
 (segment (start 104.14 67.40625) (end 101.39375 67.40625) (width 0.254) (layer "F.Cu") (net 2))
 (segment (start 120.44375 67.40625) (end 117.59375 64.55625) (width 0.254) (layer "F.Cu") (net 42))
 (segment (start 123.19 67.40625) (end 120.44375 67.40625) (width 0.254) (layer "F.Cu") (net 42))
 (segment (start 99.23125 54.80975) (end 100.03325 55.61175) (width 0.254) (layer "F.Cu") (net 8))
 (segment (start 99.23125 53.93475) (end 99.23125 54.80975) (width 0.254) (layer "F.Cu") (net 8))
 (segment (start 102.532 55.61175) (end 105.75625 52.3875) (width 0.254) (layer "F.Cu") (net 8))
 (segment (start 100.03325 55.61175) (end 102.532 55.61175) (width 0.254) (layer "F.Cu") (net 8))
 (segment (start 73.025 68.604868) (end 84.588882 80.16875) (width 0.254) (layer "F.Cu") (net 30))
 (segment (start 105.56875 80.9625) (end 105.56875 82.55) (width 0.254) (layer "F.Cu") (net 30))
 (segment (start 84.588882 80.16875) (end 104.775 80.16875) (width 0.254) (layer "F.Cu") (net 30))
 (segment (start 104.775 80.16875) (end 105.56875 80.9625) (width 0.254) (layer "F.Cu") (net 30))
 (segment (start 105.56875 82.55) (end 100.074259 88.044491) (width 0.254) (layer "F.Cu") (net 30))
 (segment (start 73.025 66.51625) (end 73.025 68.604868) (width 0.254) (layer "F.Cu") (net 30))
 (segment (start 104.775 81.75625) (end 103.98125 80.9625) (width 0.254) (layer "F.Cu") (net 12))
 (segment (start 104.775 82.212379) (end 104.775 81.75625) (width 0.254) (layer "F.Cu") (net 12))
 (segment (start 103.98125 80.9625) (end 97.692151 80.9625) (width 0.254) (layer "F.Cu") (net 12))
 (segment (start 99.508573 87.478806) (end 104.775 82.212379) (width 0.254) (layer "F.Cu") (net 12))
 (via (at 97.692151 80.9625) (size 0.8) (drill 0.4) (layers "F.Cu" "B.Cu") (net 12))
 (segment (start 92.23375 76.35875) (end 92.23375 66.51625) (width 0.254) (layer "B.Cu") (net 12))
 (segment (start 97.692151 80.9625) (end 96.8375 80.9625) (width 0.254) (layer "B.Cu") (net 12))
 (segment (start 96.8375 80.9625) (end 92.23375 76.35875) (width 0.254) (layer "B.Cu") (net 12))
 (segment (start 98.942888 86.794612) (end 101.6 84.1375) (width 0.254) (layer "F.Cu") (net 31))
 (segment (start 111.125 77.7875) (end 111.28375 77.62875) (width 0.254) (layer "F.Cu") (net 31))
 (segment (start 111.28375 77.62875) (end 111.28375 66.51625) (width 0.254) (layer "F.Cu") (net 31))
 (segment (start 98.942888 86.91312) (end 98.942888 86.794612) (width 0.254) (layer "F.Cu") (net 31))
 (via (at 111.125 77.7875) (size 0.8) (drill 0.4) (layers "F.Cu" "B.Cu") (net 31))
 (via (at 101.6 84.1375) (size 0.8) (drill 0.4) (layers "F.Cu" "B.Cu") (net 31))
 (segment (start 102.39375 83.34375) (end 103.1875 83.34375) (width 0.254) (layer "B.Cu") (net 31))
 (segment (start 103.1875 83.34375) (end 103.98125 84.1375) (width 0.254) (layer "B.Cu") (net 31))
 (segment (start 105.56875 88.10625) (end 111.125 82.55) (width 0.254) (layer "B.Cu") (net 31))
 (segment (start 104.775 88.10625) (end 105.56875 88.10625) (width 0.254) (layer "B.Cu") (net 31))
 (segment (start 111.125 82.55) (end 111.125 77.7875) (width 0.254) (layer "B.Cu") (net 31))
 (segment (start 103.98125 84.1375) (end 103.98125 87.3125) (width 0.254) (layer "B.Cu") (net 31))
 (segment (start 101.6 84.1375) (end 102.39375 83.34375) (width 0.254) (layer "B.Cu") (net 31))
 (segment (start 103.98125 87.3125) (end 104.775 88.10625) (width 0.254) (layer "B.Cu") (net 31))
 (segment (start 99.47375 56.35625) (end 105.45 56.35625) (width 0.254) (layer "F.Cu") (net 7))
 (segment (start 98.43125 55.31375) (end 99.47375 56.35625) (width 0.254) (layer "F.Cu") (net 7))
 (segment (start 98.43125 53.93475) (end 98.43125 55.31375) (width 0.254) (layer "F.Cu") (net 7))
 (segment (start 87.3125 97.412137) (end 90.316185 94.408452) (width 0.254) (layer "F.Cu") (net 16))
 (segment (start 87.3125 100.0125) (end 87.3125 97.412137) (width 0.254) (layer "F.Cu") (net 16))
 (segment (start 107.275 56.35625) (end 108.74375 56.35625) (width 0.254) (layer "F.Cu") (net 16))
 (segment (start 108.74375 56.35625) (end 111.125 58.7375) (width 0.254) (layer "F.Cu") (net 16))
 (segment (start 88.10625 100.80625) (end 87.3125 100.0125) (width 0.254) (layer "F.Cu") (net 16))
 (via (at 88.10625 100.80625) (size 0.8) (drill 0.4) (layers "F.Cu" "B.Cu") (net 16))
 (via (at 111.125 58.7375) (size 0.8) (drill 0.4) (layers "F.Cu" "B.Cu") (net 16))
 (segment (start 103.1875 66.675) (end 103.1875 69.85) (width 0.254) (layer "B.Cu") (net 16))
 (segment (start 103.1875 69.85) (end 99.21875 73.81875) (width 0.254) (layer "B.Cu") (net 16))
 (segment (start 111.125 58.7375) (end 103.1875 66.675) (width 0.254) (layer "B.Cu") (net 16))
 (segment (start 99.21875 89.69375) (end 88.10625 100.80625) (width 0.254) (layer "B.Cu") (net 16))
 (segment (start 99.21875 73.81875) (end 99.21875 89.69375) (width 0.254) (layer "B.Cu") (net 16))
 (segment (start 97.63125 53.93475) (end 97.63125 55.31375) (width 0.254) (layer "F.Cu") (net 6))
 (segment (start 100.70575 58.38825) (end 105.45 58.38825) (width 0.254) (layer "F.Cu") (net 6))
 (segment (start 97.63125 55.31375) (end 100.70575 58.38825) (width 0.254) (layer "F.Cu") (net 6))
 (segment (start 88.10625 97.749758) (end 90.88187 94.974138) (width 0.254) (layer "F.Cu") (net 17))
 (segment (start 107.275 58.38825) (end 109.18825 58.38825) (width 0.254) (layer "F.Cu") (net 17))
 (segment (start 88.10625 99.21875) (end 88.10625 97.749758) (width 0.254) (layer "F.Cu") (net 17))
 (segment (start 109.18825 58.38825) (end 109.5375 58.7375) (width 0.254) (layer "F.Cu") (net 17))
 (via (at 109.5375 58.7375) (size 0.8) (drill 0.4) (layers "F.Cu" "B.Cu") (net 17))
 (via (at 88.10625 99.21875) (size 0.8) (drill 0.4) (layers "F.Cu" "B.Cu") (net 17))
 (segment (start 109.5375 58.7375) (end 98.418651 69.856349) (width 0.254) (layer "B.Cu") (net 17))
 (segment (start 98.418651 69.856349) (end 98.418651 88.906349) (width 0.254) (layer "B.Cu") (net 17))
 (segment (start 98.418651 88.906349) (end 88.10625 99.21875) (width 0.254) (layer "B.Cu") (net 17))
 (segment (start 100.440322 101.172178) (end 105.714298 106.446154) (width 0.254) (layer "F.Cu") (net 4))
 (segment (start 105.714298 106.446154) (end 109.641346 106.446154) (width 0.254) (layer "F.Cu") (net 4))
 (segment (start 97.811517 98.543373) (end 100.440322 101.172178) (width 0.254) (layer "F.Cu") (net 4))
 (segment (start 97.811517 98.36825) (end 97.811517 98.543373) (width 0.254) (layer "F.Cu") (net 4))
 (segment (start 109.641346 106.446154) (end 121.36875 94.71875) (width 0.254) (layer "F.Cu") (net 4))
 (segment (start 96.95625 103.1875) (end 100.0125 103.1875) (width 0.254) (layer "F.Cu") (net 4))
 (segment (start 100.0125 103.1875) (end 100.440322 102.759678) (width 0.254) (layer "F.Cu") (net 4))
 (segment (start 100.440322 102.759678) (end 100.440322 101.172178) (width 0.254) (layer "F.Cu") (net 4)))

